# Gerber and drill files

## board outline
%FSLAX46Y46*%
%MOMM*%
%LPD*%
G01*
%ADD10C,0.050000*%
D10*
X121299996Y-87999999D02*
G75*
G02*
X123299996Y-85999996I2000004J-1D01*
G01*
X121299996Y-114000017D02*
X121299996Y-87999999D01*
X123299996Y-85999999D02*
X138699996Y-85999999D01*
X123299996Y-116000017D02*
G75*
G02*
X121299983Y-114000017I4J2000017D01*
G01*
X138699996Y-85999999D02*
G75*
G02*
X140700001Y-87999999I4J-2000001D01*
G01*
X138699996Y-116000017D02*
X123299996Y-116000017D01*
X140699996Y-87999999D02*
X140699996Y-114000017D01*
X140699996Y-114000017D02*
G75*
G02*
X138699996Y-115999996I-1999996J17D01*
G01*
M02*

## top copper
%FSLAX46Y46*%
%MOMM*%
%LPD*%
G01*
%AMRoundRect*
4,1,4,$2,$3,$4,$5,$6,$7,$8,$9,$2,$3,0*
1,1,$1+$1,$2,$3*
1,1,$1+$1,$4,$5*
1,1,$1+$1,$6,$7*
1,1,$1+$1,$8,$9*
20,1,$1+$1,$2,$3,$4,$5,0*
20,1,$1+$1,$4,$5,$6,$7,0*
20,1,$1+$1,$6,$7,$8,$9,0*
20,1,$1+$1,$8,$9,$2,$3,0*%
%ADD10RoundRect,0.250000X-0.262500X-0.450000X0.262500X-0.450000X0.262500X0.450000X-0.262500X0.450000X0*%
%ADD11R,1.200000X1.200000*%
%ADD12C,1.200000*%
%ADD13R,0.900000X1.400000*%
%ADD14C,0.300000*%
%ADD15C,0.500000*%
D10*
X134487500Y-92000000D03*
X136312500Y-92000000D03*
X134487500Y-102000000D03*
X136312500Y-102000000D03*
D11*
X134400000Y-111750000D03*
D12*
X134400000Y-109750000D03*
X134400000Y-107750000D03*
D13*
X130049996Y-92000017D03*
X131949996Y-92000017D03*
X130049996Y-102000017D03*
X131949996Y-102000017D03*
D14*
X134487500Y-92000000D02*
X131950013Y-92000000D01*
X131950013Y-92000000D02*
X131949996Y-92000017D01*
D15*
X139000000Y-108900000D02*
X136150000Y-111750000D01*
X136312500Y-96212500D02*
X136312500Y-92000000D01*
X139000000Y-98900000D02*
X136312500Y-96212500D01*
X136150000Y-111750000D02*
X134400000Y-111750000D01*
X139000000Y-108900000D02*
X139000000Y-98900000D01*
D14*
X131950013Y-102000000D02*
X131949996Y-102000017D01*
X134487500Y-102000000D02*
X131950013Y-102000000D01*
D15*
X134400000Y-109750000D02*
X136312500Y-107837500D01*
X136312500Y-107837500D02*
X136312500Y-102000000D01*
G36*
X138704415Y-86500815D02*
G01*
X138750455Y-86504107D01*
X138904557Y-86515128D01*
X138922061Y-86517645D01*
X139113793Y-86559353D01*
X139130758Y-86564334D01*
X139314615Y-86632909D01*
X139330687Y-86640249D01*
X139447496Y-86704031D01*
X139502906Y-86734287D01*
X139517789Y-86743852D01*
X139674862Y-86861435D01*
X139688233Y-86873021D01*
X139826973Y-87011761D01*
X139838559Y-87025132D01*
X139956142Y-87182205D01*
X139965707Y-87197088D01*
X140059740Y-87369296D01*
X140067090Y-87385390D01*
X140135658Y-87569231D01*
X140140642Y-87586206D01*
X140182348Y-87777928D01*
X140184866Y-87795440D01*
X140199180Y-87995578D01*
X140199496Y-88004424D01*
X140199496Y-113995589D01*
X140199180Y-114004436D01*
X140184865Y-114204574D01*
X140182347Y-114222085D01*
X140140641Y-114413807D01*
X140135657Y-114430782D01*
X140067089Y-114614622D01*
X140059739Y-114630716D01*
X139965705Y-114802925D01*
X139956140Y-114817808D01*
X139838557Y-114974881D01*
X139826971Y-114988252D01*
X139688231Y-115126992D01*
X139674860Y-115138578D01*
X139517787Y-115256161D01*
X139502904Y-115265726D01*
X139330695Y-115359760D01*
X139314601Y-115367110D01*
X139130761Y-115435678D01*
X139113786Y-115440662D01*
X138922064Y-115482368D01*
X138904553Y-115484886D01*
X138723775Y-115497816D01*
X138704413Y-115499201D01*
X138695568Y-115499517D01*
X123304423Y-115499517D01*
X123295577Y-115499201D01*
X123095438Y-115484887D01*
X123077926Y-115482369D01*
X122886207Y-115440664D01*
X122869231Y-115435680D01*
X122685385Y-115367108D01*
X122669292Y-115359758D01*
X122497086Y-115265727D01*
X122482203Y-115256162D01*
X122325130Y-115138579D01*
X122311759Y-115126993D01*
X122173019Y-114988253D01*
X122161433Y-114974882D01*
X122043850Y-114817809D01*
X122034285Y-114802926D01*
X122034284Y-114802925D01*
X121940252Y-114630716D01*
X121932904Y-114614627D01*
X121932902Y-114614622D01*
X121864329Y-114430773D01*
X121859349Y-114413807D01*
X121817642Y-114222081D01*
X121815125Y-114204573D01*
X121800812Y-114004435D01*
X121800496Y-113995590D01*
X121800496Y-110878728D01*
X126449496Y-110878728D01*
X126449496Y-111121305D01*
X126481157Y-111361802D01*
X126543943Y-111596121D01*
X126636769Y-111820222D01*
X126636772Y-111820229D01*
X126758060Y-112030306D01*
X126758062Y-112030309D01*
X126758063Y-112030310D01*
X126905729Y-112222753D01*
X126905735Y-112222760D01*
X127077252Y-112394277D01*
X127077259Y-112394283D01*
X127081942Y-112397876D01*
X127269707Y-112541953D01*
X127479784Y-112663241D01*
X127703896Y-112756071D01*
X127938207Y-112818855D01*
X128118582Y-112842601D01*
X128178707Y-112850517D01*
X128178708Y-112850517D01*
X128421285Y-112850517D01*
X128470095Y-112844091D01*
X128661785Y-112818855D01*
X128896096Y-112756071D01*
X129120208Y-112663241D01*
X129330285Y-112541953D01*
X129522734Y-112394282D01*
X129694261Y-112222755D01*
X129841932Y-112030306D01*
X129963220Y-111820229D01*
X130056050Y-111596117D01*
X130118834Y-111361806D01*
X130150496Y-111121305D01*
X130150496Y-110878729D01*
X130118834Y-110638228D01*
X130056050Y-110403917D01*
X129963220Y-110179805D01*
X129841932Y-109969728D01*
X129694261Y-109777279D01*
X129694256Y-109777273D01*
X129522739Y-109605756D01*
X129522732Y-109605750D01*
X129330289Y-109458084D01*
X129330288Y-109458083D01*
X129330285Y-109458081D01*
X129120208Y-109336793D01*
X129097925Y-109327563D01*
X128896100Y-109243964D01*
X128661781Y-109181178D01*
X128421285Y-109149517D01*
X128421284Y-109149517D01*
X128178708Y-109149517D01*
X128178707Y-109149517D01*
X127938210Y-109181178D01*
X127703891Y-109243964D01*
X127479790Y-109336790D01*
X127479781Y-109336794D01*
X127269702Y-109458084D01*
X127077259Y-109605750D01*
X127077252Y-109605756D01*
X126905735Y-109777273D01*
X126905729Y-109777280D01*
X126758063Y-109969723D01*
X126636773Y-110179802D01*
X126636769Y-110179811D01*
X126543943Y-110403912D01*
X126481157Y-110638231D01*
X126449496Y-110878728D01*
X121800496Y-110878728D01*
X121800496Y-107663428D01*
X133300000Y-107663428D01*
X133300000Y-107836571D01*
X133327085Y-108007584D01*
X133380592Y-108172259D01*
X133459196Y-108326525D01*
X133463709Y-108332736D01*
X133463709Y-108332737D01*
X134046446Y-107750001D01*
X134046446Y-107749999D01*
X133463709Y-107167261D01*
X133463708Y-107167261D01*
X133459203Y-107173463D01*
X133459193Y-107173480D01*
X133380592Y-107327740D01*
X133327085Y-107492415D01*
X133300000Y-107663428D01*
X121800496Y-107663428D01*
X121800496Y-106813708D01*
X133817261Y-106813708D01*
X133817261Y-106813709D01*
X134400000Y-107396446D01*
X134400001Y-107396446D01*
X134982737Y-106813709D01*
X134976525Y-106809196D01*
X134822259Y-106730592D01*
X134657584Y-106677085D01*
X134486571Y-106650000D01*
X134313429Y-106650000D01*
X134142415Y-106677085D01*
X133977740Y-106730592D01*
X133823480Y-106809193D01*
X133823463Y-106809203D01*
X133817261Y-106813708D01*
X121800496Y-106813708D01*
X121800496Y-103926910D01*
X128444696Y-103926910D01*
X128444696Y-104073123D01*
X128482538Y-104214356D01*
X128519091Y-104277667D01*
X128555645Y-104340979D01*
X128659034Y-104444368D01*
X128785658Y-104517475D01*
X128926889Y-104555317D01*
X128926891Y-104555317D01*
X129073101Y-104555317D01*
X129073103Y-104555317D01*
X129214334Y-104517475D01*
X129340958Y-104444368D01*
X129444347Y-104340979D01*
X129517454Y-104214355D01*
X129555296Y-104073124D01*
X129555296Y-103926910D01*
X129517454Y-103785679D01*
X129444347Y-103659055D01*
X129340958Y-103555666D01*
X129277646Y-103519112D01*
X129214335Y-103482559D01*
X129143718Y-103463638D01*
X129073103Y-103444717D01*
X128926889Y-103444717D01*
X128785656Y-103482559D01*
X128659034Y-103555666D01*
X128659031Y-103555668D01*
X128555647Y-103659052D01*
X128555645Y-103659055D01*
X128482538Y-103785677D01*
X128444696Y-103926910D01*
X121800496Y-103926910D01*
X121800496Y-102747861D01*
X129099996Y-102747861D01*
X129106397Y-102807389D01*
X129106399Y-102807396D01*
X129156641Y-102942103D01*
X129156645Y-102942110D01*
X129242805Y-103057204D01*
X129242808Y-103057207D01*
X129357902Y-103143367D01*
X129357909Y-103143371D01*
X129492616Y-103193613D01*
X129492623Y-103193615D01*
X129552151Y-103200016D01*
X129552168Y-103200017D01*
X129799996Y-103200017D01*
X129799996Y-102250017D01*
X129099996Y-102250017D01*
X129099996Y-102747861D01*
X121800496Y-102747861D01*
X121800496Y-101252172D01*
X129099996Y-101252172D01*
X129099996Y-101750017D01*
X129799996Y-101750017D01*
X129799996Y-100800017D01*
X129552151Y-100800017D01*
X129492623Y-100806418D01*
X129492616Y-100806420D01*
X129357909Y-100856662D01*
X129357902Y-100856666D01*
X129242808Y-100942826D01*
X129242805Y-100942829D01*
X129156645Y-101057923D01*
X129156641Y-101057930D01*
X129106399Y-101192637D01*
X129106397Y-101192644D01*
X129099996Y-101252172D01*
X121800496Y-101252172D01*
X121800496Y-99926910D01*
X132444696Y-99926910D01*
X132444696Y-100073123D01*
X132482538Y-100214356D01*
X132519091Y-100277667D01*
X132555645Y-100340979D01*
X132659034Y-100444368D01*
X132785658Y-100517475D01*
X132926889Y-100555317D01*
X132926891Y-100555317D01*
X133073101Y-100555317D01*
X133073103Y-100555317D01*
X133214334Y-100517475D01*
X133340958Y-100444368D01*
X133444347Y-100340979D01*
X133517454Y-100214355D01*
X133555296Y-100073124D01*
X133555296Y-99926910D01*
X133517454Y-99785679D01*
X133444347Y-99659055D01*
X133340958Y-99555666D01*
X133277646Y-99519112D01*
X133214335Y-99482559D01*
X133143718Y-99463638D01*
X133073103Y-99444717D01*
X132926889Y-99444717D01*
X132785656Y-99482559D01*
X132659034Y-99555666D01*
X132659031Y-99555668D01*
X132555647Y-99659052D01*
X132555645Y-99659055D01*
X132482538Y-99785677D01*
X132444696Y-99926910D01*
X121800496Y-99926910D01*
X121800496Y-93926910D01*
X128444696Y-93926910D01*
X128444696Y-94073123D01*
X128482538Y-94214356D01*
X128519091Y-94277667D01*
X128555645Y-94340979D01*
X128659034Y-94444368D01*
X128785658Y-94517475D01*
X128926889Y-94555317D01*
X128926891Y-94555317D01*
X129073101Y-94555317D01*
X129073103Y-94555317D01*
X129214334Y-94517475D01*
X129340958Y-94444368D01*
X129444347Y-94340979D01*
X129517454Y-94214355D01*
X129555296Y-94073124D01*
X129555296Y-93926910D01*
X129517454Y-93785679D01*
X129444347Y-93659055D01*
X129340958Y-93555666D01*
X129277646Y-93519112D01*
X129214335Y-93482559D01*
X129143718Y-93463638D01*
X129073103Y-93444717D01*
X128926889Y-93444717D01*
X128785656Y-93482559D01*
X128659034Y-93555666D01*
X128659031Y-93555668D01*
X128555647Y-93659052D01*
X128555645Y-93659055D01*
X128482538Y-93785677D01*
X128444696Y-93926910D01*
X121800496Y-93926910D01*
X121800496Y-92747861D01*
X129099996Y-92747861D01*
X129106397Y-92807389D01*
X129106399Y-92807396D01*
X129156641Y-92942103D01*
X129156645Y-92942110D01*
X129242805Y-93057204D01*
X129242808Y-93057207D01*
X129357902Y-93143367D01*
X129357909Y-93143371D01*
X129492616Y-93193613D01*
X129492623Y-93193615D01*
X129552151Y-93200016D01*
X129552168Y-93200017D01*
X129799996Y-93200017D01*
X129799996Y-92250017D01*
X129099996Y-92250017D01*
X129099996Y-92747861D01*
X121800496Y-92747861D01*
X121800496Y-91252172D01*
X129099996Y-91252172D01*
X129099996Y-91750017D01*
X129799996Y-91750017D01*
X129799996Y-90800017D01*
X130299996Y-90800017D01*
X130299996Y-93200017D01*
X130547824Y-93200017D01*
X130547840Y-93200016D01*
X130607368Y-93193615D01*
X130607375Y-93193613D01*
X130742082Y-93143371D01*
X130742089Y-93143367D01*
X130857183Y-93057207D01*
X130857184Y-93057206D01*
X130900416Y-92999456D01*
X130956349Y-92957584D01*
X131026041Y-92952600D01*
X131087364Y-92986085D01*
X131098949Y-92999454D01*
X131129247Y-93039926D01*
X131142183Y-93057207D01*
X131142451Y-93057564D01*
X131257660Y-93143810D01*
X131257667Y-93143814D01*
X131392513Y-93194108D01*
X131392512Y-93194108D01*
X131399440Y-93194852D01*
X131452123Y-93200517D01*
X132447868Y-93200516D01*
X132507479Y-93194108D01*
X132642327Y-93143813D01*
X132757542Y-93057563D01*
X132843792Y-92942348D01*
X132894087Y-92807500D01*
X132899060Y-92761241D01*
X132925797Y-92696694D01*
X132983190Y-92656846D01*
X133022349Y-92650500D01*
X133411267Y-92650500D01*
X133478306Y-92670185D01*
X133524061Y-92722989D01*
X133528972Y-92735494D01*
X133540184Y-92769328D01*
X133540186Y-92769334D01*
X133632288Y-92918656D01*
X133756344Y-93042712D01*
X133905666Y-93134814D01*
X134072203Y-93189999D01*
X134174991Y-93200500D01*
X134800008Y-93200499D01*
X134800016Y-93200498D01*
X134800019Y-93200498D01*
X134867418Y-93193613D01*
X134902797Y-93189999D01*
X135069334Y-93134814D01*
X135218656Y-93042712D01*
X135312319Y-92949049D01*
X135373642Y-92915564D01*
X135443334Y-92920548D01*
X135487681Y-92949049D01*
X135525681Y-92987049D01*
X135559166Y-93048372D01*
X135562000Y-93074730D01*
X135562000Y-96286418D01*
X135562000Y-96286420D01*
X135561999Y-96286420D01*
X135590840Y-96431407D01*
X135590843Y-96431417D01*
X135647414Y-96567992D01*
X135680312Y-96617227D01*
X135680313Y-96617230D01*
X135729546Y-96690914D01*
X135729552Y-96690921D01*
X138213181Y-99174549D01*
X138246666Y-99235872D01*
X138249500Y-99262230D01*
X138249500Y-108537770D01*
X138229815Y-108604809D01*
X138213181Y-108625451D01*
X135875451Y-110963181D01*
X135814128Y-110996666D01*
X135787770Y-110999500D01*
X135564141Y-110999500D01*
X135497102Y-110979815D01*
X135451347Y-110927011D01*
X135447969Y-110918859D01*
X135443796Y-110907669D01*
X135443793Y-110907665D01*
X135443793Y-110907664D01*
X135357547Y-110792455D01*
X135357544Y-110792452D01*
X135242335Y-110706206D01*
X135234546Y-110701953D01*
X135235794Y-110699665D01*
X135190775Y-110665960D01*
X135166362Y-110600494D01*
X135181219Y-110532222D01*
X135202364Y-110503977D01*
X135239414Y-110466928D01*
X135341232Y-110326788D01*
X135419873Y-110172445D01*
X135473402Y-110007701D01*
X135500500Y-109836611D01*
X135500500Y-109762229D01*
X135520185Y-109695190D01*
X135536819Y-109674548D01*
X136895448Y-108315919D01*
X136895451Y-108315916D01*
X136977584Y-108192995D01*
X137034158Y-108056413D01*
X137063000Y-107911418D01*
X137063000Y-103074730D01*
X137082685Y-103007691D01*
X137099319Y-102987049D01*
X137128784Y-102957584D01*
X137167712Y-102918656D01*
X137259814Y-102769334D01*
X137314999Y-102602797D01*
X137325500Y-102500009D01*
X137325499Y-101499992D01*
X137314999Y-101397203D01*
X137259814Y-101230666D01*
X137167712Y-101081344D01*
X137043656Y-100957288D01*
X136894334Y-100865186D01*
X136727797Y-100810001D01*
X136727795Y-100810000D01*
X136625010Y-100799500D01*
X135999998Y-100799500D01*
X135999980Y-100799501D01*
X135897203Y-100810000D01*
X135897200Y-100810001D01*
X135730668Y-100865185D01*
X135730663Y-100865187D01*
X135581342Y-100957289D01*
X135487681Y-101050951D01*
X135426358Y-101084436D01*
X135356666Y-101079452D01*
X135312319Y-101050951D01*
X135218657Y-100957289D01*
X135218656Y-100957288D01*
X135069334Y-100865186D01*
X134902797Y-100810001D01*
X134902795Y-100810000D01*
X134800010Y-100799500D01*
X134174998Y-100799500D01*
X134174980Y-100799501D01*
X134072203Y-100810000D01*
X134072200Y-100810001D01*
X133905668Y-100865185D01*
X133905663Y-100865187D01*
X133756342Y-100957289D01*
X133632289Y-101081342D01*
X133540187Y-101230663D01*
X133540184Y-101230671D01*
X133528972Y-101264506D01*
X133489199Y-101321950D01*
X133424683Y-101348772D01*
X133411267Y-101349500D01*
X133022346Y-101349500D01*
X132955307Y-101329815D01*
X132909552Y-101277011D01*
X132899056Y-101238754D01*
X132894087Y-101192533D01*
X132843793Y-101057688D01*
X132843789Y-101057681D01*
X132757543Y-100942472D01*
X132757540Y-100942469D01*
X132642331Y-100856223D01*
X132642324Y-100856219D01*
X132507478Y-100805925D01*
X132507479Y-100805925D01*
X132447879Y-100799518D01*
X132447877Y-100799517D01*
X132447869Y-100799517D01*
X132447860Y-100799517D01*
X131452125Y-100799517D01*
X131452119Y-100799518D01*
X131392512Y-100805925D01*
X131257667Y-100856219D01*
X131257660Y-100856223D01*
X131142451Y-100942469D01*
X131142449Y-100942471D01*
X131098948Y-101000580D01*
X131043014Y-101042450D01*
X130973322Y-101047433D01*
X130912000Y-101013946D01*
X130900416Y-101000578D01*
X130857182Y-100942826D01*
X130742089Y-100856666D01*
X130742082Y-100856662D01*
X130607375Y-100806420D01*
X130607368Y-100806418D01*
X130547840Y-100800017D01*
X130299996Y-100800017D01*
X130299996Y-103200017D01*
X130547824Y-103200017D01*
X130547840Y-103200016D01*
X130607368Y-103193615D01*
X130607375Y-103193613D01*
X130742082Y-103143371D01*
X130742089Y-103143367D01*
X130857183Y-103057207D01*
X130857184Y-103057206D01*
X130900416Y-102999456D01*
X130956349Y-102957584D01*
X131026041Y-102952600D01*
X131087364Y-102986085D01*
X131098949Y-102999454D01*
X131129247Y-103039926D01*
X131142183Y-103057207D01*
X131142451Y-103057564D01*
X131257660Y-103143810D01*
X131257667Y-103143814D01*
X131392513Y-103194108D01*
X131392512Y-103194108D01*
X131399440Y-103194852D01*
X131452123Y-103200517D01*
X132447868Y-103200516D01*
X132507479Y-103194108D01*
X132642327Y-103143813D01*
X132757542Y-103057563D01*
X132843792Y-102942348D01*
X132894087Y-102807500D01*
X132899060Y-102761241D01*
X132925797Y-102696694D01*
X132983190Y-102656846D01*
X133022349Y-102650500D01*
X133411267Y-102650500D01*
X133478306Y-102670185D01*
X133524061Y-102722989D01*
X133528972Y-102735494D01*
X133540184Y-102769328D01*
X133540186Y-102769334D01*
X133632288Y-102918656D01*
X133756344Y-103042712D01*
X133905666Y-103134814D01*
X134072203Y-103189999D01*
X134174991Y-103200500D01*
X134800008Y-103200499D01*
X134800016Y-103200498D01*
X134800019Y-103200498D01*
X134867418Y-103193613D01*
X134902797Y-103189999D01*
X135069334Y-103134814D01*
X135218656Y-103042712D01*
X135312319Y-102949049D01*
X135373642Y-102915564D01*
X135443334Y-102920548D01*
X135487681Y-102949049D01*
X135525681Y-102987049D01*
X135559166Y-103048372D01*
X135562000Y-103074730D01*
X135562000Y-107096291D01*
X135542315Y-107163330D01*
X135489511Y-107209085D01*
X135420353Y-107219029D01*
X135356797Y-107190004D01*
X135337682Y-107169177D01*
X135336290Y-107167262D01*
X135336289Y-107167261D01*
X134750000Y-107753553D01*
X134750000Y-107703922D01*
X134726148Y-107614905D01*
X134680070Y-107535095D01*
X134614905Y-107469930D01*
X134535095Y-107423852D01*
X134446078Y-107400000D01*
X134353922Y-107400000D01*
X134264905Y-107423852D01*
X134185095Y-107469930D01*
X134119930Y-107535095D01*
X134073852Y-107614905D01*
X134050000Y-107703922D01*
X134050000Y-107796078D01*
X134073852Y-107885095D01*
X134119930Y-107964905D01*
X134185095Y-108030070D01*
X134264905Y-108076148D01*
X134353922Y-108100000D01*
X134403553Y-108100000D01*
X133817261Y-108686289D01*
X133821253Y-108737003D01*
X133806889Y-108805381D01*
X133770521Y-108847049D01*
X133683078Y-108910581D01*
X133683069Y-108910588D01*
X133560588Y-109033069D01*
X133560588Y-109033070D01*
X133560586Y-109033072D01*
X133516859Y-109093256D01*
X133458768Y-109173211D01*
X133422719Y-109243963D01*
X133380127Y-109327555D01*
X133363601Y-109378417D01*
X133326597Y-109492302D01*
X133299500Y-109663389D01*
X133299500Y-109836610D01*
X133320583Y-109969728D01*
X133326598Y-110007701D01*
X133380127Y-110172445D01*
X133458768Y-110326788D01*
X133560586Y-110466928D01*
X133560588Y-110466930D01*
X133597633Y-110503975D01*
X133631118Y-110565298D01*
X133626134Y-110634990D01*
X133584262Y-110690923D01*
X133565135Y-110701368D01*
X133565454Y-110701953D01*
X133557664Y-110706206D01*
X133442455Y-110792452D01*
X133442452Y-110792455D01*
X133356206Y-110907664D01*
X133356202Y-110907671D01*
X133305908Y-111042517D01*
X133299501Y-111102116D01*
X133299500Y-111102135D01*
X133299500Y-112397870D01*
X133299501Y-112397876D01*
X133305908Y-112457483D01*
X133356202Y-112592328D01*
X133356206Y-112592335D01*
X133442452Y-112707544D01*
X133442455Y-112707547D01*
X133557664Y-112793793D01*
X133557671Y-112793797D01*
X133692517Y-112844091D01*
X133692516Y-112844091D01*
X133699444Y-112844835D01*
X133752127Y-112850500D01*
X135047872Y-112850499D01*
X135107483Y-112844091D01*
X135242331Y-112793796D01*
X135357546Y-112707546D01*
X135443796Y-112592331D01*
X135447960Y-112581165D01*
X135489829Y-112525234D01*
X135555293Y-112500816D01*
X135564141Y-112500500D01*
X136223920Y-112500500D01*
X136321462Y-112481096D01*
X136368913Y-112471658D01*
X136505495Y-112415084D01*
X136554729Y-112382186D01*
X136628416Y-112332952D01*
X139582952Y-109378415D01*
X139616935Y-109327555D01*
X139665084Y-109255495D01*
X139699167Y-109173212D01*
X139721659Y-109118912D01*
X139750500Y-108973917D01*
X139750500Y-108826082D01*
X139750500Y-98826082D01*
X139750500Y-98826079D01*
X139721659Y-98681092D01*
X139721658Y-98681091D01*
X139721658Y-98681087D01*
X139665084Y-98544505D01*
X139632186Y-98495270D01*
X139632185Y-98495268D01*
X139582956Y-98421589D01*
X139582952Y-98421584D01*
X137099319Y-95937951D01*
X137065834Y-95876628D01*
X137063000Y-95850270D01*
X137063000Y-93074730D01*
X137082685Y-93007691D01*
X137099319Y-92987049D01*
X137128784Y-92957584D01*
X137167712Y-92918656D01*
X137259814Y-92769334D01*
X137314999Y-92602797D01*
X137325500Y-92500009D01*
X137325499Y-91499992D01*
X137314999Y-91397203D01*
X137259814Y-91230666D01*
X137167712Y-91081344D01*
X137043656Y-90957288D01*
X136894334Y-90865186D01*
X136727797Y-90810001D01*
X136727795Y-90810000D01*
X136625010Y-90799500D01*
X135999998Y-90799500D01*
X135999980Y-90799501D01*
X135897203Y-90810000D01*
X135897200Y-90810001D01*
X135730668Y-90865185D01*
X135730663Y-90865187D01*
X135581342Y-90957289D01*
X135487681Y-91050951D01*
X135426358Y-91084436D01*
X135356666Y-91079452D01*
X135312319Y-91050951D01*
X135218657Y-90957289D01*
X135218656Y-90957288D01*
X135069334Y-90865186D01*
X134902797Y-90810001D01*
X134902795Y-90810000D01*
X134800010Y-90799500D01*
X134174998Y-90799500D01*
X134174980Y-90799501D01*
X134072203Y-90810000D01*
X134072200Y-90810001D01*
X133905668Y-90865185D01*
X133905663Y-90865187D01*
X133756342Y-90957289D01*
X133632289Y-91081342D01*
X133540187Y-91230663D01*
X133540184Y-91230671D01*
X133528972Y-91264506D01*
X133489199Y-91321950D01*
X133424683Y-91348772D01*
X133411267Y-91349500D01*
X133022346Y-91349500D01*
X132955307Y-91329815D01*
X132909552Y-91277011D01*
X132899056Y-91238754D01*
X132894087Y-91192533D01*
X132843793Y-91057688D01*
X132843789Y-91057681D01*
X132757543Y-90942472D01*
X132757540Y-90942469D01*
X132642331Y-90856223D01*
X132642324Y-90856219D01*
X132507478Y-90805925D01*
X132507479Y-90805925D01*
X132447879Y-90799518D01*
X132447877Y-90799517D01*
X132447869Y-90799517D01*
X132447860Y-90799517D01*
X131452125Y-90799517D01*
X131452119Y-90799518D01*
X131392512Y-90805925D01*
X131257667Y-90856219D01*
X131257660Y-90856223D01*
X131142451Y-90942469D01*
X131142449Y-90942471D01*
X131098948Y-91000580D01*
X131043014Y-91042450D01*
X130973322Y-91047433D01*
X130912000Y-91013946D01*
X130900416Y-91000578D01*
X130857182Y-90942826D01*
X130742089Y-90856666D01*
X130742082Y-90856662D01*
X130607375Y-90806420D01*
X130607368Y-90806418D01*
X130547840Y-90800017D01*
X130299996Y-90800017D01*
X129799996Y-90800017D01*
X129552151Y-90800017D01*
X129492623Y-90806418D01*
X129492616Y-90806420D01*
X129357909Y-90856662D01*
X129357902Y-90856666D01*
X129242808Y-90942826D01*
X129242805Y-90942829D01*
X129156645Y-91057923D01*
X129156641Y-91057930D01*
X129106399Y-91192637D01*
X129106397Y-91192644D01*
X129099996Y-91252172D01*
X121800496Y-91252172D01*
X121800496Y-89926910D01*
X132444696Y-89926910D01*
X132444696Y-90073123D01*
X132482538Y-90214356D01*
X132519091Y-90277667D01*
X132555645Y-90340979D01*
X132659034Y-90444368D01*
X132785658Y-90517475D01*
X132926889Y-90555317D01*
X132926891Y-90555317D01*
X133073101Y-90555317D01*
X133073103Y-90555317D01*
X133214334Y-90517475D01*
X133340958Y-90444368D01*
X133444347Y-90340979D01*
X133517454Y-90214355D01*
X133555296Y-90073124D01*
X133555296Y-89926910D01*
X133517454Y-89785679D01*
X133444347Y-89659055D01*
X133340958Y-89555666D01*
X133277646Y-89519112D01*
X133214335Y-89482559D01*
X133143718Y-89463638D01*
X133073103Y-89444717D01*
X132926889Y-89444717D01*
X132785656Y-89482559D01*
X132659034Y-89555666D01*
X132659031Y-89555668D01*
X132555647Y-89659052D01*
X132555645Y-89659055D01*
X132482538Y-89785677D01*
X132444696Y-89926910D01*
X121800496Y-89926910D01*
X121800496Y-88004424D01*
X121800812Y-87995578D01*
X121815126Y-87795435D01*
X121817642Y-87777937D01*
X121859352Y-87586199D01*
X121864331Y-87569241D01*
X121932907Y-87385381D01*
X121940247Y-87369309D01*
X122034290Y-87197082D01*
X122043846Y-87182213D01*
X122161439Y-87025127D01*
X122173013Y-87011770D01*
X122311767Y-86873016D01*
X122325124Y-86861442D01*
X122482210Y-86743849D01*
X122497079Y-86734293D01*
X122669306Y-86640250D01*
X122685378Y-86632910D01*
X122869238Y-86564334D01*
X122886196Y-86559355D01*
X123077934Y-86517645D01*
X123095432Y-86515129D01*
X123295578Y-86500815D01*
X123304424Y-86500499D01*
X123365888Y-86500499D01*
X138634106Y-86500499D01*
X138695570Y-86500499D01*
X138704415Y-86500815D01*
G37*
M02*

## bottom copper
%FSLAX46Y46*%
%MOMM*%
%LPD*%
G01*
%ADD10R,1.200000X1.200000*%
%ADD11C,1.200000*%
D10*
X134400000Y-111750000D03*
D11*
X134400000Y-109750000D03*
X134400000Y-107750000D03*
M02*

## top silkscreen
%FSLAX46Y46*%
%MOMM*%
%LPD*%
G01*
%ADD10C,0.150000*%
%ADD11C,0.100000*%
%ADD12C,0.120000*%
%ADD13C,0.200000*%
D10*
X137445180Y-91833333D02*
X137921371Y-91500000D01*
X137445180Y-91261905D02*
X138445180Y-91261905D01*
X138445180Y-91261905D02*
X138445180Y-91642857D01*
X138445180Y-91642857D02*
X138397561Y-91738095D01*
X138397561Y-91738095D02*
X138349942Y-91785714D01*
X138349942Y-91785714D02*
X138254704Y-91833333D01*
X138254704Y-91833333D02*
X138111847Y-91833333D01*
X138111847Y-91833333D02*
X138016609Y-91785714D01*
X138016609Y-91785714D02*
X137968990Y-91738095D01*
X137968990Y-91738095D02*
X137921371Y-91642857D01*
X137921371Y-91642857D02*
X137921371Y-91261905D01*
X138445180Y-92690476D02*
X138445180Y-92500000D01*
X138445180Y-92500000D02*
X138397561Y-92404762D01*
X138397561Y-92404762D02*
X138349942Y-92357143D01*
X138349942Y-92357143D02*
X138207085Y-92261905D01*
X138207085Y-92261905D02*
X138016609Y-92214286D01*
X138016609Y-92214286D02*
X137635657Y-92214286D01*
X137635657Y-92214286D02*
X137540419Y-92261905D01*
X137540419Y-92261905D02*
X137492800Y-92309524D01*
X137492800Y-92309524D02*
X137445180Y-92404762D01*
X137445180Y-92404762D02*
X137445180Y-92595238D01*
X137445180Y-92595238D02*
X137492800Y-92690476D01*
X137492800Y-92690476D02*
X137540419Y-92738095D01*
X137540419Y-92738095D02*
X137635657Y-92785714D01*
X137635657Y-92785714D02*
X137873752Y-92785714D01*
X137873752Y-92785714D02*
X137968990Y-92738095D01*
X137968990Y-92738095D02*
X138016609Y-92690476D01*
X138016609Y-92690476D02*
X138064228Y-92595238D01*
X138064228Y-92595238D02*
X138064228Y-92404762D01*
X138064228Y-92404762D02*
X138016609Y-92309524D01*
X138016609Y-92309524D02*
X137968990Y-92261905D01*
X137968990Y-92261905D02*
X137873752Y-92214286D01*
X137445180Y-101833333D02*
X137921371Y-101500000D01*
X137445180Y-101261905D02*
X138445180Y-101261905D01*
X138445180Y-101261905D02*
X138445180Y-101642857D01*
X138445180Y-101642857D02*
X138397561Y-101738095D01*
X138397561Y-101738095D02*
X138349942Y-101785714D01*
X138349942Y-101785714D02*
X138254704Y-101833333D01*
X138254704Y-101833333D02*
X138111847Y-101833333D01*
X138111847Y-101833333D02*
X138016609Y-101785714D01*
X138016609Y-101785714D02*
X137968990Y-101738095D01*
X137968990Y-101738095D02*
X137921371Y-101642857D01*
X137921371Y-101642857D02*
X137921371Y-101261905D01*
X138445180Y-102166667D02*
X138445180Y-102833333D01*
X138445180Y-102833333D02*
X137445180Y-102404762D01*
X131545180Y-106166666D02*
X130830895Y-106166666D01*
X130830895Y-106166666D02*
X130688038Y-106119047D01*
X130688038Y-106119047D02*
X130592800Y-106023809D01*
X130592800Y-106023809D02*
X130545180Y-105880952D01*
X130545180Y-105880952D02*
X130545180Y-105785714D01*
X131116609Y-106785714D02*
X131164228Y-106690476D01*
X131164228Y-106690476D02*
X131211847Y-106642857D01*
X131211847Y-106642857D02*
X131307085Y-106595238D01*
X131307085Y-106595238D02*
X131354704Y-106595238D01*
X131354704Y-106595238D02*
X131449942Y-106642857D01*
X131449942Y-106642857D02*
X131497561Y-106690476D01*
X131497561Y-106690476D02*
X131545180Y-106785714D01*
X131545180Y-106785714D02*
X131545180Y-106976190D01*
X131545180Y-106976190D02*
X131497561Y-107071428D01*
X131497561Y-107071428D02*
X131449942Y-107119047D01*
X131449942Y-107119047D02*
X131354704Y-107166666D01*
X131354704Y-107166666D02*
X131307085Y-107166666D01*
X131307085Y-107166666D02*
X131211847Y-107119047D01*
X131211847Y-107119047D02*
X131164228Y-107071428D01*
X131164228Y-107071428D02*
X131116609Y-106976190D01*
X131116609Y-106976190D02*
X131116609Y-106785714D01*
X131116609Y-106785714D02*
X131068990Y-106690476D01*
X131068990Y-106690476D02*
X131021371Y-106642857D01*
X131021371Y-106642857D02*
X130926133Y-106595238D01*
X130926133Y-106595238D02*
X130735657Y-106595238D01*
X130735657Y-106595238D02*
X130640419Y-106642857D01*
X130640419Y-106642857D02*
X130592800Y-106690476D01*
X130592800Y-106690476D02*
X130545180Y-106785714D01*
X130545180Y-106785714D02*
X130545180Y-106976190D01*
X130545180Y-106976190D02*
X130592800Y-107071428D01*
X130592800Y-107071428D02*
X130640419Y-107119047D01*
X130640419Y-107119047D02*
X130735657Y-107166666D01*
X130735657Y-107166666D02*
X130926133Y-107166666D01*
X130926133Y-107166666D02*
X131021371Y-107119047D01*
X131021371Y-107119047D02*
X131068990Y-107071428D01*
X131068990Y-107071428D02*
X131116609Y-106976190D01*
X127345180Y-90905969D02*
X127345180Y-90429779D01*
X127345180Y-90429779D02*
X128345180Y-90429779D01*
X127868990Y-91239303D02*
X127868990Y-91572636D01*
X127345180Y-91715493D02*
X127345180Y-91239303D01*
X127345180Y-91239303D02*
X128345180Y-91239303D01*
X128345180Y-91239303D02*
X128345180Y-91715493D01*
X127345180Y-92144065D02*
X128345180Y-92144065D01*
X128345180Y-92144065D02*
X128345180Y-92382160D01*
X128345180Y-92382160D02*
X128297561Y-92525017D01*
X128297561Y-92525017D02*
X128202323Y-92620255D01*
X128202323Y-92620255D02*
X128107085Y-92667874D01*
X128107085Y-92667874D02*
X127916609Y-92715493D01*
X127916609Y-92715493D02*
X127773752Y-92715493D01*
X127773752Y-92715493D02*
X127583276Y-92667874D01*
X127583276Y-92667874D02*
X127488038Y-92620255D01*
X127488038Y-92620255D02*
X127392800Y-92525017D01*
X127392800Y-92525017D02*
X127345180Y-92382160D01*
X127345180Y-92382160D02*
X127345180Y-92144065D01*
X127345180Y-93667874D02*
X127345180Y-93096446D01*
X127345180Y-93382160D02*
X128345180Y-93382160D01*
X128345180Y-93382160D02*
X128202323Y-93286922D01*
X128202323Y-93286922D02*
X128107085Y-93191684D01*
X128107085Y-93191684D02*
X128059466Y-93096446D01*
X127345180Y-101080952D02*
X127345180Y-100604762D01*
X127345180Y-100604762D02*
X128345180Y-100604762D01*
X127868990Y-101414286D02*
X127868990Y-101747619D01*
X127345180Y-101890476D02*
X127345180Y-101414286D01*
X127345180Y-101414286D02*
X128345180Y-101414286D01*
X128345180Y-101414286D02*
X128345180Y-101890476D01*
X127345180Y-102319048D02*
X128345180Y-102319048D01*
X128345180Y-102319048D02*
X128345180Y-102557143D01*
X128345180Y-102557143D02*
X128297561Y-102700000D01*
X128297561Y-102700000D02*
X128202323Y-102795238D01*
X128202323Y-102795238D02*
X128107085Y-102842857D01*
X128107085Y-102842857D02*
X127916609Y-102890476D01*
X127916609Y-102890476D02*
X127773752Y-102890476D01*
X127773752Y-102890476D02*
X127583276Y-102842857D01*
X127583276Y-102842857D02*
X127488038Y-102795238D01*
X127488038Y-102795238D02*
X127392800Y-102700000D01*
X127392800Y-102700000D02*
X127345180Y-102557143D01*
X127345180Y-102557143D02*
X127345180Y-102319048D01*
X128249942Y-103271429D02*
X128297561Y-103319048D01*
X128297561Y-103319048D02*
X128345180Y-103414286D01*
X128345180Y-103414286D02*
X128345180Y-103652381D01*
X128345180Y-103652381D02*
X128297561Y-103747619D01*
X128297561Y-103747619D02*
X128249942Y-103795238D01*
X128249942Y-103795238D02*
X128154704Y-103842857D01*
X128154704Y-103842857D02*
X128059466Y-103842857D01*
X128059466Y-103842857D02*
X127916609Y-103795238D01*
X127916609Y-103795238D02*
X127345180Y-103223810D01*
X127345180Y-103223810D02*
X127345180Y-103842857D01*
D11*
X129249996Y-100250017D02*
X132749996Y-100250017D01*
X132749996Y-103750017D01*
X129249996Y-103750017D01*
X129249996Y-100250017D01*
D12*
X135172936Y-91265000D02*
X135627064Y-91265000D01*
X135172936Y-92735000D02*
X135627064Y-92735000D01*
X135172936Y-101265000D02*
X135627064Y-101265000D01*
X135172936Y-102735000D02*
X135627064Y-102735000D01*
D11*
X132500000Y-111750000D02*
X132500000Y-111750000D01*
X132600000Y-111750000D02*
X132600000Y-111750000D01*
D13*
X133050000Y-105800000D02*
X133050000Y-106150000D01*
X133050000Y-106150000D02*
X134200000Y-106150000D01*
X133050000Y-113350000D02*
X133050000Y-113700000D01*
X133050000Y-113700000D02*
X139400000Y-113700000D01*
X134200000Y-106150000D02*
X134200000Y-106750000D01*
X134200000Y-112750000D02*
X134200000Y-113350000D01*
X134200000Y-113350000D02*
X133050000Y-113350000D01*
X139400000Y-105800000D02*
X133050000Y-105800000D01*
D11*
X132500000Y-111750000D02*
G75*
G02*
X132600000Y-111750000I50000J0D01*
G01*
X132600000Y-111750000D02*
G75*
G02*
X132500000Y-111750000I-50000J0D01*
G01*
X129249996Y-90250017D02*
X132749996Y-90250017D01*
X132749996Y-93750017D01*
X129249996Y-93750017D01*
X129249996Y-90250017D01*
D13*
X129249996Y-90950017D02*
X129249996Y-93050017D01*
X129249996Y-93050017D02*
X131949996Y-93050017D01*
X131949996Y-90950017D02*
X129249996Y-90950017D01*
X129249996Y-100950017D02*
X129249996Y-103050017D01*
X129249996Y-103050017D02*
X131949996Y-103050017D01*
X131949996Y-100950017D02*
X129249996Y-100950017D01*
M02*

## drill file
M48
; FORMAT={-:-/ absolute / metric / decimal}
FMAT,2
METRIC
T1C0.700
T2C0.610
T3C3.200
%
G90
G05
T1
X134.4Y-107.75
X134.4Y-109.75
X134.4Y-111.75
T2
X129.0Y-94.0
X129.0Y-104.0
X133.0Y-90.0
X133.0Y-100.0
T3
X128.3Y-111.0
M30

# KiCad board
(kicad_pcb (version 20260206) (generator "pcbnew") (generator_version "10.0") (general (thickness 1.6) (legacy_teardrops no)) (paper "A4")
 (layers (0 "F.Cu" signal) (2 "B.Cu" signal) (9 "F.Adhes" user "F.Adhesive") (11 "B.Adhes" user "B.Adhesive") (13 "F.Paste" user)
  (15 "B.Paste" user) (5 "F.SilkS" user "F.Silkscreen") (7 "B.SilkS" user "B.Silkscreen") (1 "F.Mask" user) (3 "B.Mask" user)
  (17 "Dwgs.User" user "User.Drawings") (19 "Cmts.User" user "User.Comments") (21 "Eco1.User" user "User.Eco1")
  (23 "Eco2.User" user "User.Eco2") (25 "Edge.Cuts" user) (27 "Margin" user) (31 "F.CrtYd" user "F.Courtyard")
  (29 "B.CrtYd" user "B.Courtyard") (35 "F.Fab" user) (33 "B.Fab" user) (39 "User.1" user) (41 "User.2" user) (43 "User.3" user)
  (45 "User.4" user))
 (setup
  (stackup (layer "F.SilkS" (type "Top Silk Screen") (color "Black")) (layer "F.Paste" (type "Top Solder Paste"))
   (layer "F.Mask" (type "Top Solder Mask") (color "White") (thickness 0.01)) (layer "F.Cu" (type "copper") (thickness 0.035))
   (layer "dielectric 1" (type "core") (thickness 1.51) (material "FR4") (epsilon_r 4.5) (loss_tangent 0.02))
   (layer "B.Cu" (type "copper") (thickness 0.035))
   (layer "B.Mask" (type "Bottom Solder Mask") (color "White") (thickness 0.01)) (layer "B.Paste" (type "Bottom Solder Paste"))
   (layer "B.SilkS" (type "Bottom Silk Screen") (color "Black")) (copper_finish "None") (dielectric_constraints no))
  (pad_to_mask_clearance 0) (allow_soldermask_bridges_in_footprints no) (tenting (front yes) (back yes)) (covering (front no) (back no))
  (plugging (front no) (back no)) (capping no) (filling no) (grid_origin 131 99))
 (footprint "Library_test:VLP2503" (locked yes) (layer "F.Cu") (at 130.999996 102.000017)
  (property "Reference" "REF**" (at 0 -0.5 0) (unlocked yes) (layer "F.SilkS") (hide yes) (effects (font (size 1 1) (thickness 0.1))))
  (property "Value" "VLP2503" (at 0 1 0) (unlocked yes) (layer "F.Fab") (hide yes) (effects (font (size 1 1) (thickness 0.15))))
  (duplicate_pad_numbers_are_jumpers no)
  (fp_rect (start -1.75 -1.75) (end 1.75 1.75) (stroke (width 0.1) (type default)) (fill no) (layer "F.SilkS"))
  (pad "" np_thru_hole circle (at -2 2) (size 0.6096 0.6096) (drill 0.6096) (layers "*.Cu" "*.Mask"))
  (pad "" np_thru_hole circle (at 2 -2) (size 0.6096 0.6096) (drill 0.6096) (layers "*.Cu" "*.Mask")))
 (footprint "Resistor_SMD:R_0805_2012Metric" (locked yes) (layer "F.Cu") (at 135.4 92)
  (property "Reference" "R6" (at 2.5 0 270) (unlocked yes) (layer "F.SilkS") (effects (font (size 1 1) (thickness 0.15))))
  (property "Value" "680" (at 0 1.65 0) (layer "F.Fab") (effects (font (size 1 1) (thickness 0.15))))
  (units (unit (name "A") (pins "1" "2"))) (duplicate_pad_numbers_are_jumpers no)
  (fp_line (start -0.227064 -0.735) (end 0.227064 -0.735) (stroke (width 0.12) (type solid)) (layer "F.SilkS"))
  (fp_line (start -0.227064 0.735) (end 0.227064 0.735) (stroke (width 0.12) (type solid)) (layer "F.SilkS"))
  (pad "1" smd roundrect (at -0.9125 0) (size 1.025 1.4) (layers "F.Cu" "F.Mask" "F.Paste") (roundrect_rratio 0.243902) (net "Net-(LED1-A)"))
  (pad "2" smd roundrect (at 0.9125 0) (size 1.025 1.4) (layers "F.Cu" "F.Mask" "F.Paste") (roundrect_rratio 0.243902) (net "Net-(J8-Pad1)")))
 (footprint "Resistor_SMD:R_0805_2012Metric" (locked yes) (layer "F.Cu") (at 135.4 102)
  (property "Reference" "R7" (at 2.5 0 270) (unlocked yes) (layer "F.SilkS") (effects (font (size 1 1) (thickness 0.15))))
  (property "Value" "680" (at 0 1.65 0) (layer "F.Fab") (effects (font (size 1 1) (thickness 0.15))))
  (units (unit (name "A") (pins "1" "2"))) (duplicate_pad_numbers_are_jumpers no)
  (fp_line (start -0.227064 -0.735) (end 0.227064 -0.735) (stroke (width 0.12) (type solid)) (layer "F.SilkS"))
  (fp_line (start -0.227064 0.735) (end 0.227064 0.735) (stroke (width 0.12) (type solid)) (layer "F.SilkS"))
  (pad "1" smd roundrect (at -0.9125 0) (size 1.025 1.4) (layers "F.Cu" "F.Mask" "F.Paste") (roundrect_rratio 0.243902) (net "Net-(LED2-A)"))
  (pad "2" smd roundrect (at 0.9125 0) (size 1.025 1.4) (layers "F.Cu" "F.Mask" "F.Paste") (roundrect_rratio 0.243902) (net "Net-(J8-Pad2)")))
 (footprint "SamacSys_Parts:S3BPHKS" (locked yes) (layer "F.Cu") (at 134.4 111.75 90)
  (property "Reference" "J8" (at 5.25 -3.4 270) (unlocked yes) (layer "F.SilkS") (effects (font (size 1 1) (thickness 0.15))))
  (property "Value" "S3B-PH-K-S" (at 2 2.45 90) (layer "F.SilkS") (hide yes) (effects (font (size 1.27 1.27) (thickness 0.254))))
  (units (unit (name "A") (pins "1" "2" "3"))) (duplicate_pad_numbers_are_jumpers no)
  (fp_line (start 0 -1.9) (end 0 -1.9) (stroke (width 0.1) (type solid)) (layer "F.SilkS"))
  (fp_line (start 0 -1.8) (end 0 -1.8) (stroke (width 0.1) (type solid)) (layer "F.SilkS"))
  (fp_line (start 5.95 -1.35) (end 5.6 -1.35) (stroke (width 0.2) (type solid)) (layer "F.SilkS"))
  (fp_line (start 5.6 -1.35) (end 5.6 -0.2) (stroke (width 0.2) (type solid)) (layer "F.SilkS"))
  (fp_line (start -1.6 -1.35) (end -1.95 -1.35) (stroke (width 0.2) (type solid)) (layer "F.SilkS"))
  (fp_line (start -1.95 -1.35) (end -1.95 5) (stroke (width 0.2) (type solid)) (layer "F.SilkS"))
  (fp_line (start 5.6 -0.2) (end 5 -0.2) (stroke (width 0.2) (type solid)) (layer "F.SilkS"))
  (fp_line (start -1 -0.2) (end -1.6 -0.2) (stroke (width 0.2) (type solid)) (layer "F.SilkS"))
  (fp_line (start -1.6 -0.2) (end -1.6 -1.35) (stroke (width 0.2) (type solid)) (layer "F.SilkS"))
  (fp_line (start 5.95 5) (end 5.95 -1.35) (stroke (width 0.2) (type solid)) (layer "F.SilkS"))
  (fp_arc (start 0 -1.9) (mid 0.05 -1.85) (end 0 -1.8) (stroke (width 0.1) (type solid)) (layer "F.SilkS"))
  (fp_arc (start 0 -1.8) (mid -0.05 -1.85) (end 0 -1.9) (stroke (width 0.1) (type solid)) (layer "F.SilkS"))
  (pad "1" thru_hole rect (at 0 0 90) (size 1.2 1.2) (drill 0.7) (layers "*.Cu" "*.Mask") (remove_unused_layers no) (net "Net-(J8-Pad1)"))
  (pad "2" thru_hole circle (at 2 0 90) (size 1.2 1.2) (drill 0.7) (layers "*.Cu" "*.Mask") (remove_unused_layers no) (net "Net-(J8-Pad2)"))
  (pad "3" thru_hole circle (at 4 0 90) (size 1.2 1.2) (drill 0.7) (layers "*.Cu" "*.Mask") (remove_unused_layers no) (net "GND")))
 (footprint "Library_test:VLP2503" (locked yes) (layer "F.Cu") (at 130.999996 92.000017)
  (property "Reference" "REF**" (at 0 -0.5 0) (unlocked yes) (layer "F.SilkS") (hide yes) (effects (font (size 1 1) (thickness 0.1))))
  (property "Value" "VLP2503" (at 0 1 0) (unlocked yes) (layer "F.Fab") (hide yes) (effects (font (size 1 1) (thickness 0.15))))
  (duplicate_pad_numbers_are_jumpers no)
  (fp_rect (start -1.75 -1.75) (end 1.75 1.75) (stroke (width 0.1) (type default)) (fill no) (layer "F.SilkS"))
  (pad "" np_thru_hole circle (at -2 2) (size 0.6096 0.6096) (drill 0.6096) (layers "*.Cu" "*.Mask"))
  (pad "" np_thru_hole circle (at 2 -2) (size 0.6096 0.6096) (drill 0.6096) (layers "*.Cu" "*.Mask")))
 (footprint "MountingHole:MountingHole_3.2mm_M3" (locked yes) (layer "F.Cu") (at 128.299996 111.000017)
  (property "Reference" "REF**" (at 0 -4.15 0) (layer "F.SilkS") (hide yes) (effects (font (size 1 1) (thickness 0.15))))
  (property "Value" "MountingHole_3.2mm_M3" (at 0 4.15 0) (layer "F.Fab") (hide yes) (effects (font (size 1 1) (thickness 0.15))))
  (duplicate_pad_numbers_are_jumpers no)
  (pad "" np_thru_hole circle (at 0 0) (size 3.2 3.2) (drill 3.2) (layers "*.Cu" "*.Mask")))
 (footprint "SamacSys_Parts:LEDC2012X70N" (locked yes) (layer "F.Cu") (at 130.999996 92.000017)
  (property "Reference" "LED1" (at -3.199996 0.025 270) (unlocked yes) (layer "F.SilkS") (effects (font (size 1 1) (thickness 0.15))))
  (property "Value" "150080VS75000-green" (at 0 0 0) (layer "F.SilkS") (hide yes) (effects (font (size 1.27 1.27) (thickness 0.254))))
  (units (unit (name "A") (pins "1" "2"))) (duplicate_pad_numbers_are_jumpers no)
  (fp_line (start -1.75 -1.05) (end -1.75 1.05) (stroke (width 0.2) (type solid)) (layer "F.SilkS"))
  (fp_line (start -1.75 1.05) (end 0.95 1.05) (stroke (width 0.2) (type solid)) (layer "F.SilkS"))
  (fp_line (start 0.95 -1.05) (end -1.75 -1.05) (stroke (width 0.2) (type solid)) (layer "F.SilkS"))
  (pad "1" smd rect (at -0.95 0) (size 0.9 1.4) (layers "F.Cu" "F.Mask" "F.Paste") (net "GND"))
  (pad "2" smd rect (at 0.95 0) (size 0.9 1.4) (layers "F.Cu" "F.Mask" "F.Paste") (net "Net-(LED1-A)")))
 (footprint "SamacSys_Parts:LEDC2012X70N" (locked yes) (layer "F.Cu") (at 130.999996 102.000017)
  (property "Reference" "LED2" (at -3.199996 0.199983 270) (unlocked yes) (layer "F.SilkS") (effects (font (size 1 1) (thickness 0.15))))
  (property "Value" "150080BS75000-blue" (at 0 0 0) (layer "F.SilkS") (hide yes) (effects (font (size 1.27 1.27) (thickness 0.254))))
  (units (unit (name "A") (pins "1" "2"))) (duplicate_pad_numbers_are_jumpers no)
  (fp_line (start -1.75 -1.05) (end -1.75 1.05) (stroke (width 0.2) (type solid)) (layer "F.SilkS"))
  (fp_line (start -1.75 1.05) (end 0.95 1.05) (stroke (width 0.2) (type solid)) (layer "F.SilkS"))
  (fp_line (start 0.95 -1.05) (end -1.75 -1.05) (stroke (width 0.2) (type solid)) (layer "F.SilkS"))
  (pad "1" smd rect (at -0.95 0) (size 0.9 1.4) (layers "F.Cu" "F.Mask" "F.Paste") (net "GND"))
  (pad "2" smd rect (at 0.95 0) (size 0.9 1.4) (layers "F.Cu" "F.Mask" "F.Paste") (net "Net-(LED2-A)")))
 (gr_arc (start 121.299996 87.999999) (mid 121.885782 86.585785) (end 123.299996 85.999999) (stroke (width 0.05) (type default))
  (locked yes) (layer "Edge.Cuts"))
 (gr_line (start 121.299996 114.000017) (end 121.299996 87.999999) (stroke (width 0.05) (type default)) (locked yes) (layer "Edge.Cuts"))
 (gr_line (start 123.299996 85.999999) (end 138.699996 85.999999) (stroke (width 0.05) (type default)) (locked yes) (layer "Edge.Cuts"))
 (gr_arc (start 123.299996 116.000017) (mid 121.885779 115.41423) (end 121.299996 114.000017) (stroke (width 0.05) (type default))
  (locked yes) (layer "Edge.Cuts"))
 (gr_arc (start 138.699996 85.999999) (mid 140.114213 86.585784) (end 140.699996 87.999999) (stroke (width 0.05) (type default))
  (locked yes) (layer "Edge.Cuts"))
 (gr_line (start 138.699996 116.000017) (end 123.299996 116.000017) (stroke (width 0.05) (type default)) (locked yes) (layer "Edge.Cuts"))
 (gr_line (start 140.699996 87.999999) (end 140.699996 114.000017) (stroke (width 0.05) (type default)) (locked yes) (layer "Edge.Cuts"))
 (gr_arc (start 140.699996 114.000017) (mid 140.11421 115.414231) (end 138.699996 116.000017) (stroke (width 0.05) (type default))
  (locked yes) (layer "Edge.Cuts"))
 (segment (start 134.4875 92) (end 131.950013 92) (width 0.3) (locked yes) (layer "F.Cu") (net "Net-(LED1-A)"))
 (segment (start 131.950013 92) (end 131.949996 92.000017) (width 0.3) (locked yes) (layer "F.Cu") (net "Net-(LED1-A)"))
 (segment (start 139 108.9) (end 136.15 111.75) (width 0.5) (locked yes) (layer "F.Cu") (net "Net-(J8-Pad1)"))
 (segment (start 136.3125 96.2125) (end 136.3125 92) (width 0.5) (locked yes) (layer "F.Cu") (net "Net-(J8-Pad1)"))
 (segment (start 139 98.9) (end 136.3125 96.2125) (width 0.5) (locked yes) (layer "F.Cu") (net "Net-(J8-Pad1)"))
 (segment (start 136.15 111.75) (end 134.4 111.75) (width 0.5) (locked yes) (layer "F.Cu") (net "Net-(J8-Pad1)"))
 (segment (start 139 108.9) (end 139 98.9) (width 0.5) (locked yes) (layer "F.Cu") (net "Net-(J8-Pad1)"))
 (segment (start 131.950013 102) (end 131.949996 102.000017) (width 0.3) (locked yes) (layer "F.Cu") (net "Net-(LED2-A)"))
 (segment (start 134.4875 102) (end 131.950013 102) (width 0.3) (locked yes) (layer "F.Cu") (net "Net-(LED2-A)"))
 (segment (start 134.4 109.75) (end 136.3125 107.8375) (width 0.5) (locked yes) (layer "F.Cu") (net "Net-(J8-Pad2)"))
 (segment (start 136.3125 107.8375) (end 136.3125 102) (width 0.5) (locked yes) (layer "F.Cu") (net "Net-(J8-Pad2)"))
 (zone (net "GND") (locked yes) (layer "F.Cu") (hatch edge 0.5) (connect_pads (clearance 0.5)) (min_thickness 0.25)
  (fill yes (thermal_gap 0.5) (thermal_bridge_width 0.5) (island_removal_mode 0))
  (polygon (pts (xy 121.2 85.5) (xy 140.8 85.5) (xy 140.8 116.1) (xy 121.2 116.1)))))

